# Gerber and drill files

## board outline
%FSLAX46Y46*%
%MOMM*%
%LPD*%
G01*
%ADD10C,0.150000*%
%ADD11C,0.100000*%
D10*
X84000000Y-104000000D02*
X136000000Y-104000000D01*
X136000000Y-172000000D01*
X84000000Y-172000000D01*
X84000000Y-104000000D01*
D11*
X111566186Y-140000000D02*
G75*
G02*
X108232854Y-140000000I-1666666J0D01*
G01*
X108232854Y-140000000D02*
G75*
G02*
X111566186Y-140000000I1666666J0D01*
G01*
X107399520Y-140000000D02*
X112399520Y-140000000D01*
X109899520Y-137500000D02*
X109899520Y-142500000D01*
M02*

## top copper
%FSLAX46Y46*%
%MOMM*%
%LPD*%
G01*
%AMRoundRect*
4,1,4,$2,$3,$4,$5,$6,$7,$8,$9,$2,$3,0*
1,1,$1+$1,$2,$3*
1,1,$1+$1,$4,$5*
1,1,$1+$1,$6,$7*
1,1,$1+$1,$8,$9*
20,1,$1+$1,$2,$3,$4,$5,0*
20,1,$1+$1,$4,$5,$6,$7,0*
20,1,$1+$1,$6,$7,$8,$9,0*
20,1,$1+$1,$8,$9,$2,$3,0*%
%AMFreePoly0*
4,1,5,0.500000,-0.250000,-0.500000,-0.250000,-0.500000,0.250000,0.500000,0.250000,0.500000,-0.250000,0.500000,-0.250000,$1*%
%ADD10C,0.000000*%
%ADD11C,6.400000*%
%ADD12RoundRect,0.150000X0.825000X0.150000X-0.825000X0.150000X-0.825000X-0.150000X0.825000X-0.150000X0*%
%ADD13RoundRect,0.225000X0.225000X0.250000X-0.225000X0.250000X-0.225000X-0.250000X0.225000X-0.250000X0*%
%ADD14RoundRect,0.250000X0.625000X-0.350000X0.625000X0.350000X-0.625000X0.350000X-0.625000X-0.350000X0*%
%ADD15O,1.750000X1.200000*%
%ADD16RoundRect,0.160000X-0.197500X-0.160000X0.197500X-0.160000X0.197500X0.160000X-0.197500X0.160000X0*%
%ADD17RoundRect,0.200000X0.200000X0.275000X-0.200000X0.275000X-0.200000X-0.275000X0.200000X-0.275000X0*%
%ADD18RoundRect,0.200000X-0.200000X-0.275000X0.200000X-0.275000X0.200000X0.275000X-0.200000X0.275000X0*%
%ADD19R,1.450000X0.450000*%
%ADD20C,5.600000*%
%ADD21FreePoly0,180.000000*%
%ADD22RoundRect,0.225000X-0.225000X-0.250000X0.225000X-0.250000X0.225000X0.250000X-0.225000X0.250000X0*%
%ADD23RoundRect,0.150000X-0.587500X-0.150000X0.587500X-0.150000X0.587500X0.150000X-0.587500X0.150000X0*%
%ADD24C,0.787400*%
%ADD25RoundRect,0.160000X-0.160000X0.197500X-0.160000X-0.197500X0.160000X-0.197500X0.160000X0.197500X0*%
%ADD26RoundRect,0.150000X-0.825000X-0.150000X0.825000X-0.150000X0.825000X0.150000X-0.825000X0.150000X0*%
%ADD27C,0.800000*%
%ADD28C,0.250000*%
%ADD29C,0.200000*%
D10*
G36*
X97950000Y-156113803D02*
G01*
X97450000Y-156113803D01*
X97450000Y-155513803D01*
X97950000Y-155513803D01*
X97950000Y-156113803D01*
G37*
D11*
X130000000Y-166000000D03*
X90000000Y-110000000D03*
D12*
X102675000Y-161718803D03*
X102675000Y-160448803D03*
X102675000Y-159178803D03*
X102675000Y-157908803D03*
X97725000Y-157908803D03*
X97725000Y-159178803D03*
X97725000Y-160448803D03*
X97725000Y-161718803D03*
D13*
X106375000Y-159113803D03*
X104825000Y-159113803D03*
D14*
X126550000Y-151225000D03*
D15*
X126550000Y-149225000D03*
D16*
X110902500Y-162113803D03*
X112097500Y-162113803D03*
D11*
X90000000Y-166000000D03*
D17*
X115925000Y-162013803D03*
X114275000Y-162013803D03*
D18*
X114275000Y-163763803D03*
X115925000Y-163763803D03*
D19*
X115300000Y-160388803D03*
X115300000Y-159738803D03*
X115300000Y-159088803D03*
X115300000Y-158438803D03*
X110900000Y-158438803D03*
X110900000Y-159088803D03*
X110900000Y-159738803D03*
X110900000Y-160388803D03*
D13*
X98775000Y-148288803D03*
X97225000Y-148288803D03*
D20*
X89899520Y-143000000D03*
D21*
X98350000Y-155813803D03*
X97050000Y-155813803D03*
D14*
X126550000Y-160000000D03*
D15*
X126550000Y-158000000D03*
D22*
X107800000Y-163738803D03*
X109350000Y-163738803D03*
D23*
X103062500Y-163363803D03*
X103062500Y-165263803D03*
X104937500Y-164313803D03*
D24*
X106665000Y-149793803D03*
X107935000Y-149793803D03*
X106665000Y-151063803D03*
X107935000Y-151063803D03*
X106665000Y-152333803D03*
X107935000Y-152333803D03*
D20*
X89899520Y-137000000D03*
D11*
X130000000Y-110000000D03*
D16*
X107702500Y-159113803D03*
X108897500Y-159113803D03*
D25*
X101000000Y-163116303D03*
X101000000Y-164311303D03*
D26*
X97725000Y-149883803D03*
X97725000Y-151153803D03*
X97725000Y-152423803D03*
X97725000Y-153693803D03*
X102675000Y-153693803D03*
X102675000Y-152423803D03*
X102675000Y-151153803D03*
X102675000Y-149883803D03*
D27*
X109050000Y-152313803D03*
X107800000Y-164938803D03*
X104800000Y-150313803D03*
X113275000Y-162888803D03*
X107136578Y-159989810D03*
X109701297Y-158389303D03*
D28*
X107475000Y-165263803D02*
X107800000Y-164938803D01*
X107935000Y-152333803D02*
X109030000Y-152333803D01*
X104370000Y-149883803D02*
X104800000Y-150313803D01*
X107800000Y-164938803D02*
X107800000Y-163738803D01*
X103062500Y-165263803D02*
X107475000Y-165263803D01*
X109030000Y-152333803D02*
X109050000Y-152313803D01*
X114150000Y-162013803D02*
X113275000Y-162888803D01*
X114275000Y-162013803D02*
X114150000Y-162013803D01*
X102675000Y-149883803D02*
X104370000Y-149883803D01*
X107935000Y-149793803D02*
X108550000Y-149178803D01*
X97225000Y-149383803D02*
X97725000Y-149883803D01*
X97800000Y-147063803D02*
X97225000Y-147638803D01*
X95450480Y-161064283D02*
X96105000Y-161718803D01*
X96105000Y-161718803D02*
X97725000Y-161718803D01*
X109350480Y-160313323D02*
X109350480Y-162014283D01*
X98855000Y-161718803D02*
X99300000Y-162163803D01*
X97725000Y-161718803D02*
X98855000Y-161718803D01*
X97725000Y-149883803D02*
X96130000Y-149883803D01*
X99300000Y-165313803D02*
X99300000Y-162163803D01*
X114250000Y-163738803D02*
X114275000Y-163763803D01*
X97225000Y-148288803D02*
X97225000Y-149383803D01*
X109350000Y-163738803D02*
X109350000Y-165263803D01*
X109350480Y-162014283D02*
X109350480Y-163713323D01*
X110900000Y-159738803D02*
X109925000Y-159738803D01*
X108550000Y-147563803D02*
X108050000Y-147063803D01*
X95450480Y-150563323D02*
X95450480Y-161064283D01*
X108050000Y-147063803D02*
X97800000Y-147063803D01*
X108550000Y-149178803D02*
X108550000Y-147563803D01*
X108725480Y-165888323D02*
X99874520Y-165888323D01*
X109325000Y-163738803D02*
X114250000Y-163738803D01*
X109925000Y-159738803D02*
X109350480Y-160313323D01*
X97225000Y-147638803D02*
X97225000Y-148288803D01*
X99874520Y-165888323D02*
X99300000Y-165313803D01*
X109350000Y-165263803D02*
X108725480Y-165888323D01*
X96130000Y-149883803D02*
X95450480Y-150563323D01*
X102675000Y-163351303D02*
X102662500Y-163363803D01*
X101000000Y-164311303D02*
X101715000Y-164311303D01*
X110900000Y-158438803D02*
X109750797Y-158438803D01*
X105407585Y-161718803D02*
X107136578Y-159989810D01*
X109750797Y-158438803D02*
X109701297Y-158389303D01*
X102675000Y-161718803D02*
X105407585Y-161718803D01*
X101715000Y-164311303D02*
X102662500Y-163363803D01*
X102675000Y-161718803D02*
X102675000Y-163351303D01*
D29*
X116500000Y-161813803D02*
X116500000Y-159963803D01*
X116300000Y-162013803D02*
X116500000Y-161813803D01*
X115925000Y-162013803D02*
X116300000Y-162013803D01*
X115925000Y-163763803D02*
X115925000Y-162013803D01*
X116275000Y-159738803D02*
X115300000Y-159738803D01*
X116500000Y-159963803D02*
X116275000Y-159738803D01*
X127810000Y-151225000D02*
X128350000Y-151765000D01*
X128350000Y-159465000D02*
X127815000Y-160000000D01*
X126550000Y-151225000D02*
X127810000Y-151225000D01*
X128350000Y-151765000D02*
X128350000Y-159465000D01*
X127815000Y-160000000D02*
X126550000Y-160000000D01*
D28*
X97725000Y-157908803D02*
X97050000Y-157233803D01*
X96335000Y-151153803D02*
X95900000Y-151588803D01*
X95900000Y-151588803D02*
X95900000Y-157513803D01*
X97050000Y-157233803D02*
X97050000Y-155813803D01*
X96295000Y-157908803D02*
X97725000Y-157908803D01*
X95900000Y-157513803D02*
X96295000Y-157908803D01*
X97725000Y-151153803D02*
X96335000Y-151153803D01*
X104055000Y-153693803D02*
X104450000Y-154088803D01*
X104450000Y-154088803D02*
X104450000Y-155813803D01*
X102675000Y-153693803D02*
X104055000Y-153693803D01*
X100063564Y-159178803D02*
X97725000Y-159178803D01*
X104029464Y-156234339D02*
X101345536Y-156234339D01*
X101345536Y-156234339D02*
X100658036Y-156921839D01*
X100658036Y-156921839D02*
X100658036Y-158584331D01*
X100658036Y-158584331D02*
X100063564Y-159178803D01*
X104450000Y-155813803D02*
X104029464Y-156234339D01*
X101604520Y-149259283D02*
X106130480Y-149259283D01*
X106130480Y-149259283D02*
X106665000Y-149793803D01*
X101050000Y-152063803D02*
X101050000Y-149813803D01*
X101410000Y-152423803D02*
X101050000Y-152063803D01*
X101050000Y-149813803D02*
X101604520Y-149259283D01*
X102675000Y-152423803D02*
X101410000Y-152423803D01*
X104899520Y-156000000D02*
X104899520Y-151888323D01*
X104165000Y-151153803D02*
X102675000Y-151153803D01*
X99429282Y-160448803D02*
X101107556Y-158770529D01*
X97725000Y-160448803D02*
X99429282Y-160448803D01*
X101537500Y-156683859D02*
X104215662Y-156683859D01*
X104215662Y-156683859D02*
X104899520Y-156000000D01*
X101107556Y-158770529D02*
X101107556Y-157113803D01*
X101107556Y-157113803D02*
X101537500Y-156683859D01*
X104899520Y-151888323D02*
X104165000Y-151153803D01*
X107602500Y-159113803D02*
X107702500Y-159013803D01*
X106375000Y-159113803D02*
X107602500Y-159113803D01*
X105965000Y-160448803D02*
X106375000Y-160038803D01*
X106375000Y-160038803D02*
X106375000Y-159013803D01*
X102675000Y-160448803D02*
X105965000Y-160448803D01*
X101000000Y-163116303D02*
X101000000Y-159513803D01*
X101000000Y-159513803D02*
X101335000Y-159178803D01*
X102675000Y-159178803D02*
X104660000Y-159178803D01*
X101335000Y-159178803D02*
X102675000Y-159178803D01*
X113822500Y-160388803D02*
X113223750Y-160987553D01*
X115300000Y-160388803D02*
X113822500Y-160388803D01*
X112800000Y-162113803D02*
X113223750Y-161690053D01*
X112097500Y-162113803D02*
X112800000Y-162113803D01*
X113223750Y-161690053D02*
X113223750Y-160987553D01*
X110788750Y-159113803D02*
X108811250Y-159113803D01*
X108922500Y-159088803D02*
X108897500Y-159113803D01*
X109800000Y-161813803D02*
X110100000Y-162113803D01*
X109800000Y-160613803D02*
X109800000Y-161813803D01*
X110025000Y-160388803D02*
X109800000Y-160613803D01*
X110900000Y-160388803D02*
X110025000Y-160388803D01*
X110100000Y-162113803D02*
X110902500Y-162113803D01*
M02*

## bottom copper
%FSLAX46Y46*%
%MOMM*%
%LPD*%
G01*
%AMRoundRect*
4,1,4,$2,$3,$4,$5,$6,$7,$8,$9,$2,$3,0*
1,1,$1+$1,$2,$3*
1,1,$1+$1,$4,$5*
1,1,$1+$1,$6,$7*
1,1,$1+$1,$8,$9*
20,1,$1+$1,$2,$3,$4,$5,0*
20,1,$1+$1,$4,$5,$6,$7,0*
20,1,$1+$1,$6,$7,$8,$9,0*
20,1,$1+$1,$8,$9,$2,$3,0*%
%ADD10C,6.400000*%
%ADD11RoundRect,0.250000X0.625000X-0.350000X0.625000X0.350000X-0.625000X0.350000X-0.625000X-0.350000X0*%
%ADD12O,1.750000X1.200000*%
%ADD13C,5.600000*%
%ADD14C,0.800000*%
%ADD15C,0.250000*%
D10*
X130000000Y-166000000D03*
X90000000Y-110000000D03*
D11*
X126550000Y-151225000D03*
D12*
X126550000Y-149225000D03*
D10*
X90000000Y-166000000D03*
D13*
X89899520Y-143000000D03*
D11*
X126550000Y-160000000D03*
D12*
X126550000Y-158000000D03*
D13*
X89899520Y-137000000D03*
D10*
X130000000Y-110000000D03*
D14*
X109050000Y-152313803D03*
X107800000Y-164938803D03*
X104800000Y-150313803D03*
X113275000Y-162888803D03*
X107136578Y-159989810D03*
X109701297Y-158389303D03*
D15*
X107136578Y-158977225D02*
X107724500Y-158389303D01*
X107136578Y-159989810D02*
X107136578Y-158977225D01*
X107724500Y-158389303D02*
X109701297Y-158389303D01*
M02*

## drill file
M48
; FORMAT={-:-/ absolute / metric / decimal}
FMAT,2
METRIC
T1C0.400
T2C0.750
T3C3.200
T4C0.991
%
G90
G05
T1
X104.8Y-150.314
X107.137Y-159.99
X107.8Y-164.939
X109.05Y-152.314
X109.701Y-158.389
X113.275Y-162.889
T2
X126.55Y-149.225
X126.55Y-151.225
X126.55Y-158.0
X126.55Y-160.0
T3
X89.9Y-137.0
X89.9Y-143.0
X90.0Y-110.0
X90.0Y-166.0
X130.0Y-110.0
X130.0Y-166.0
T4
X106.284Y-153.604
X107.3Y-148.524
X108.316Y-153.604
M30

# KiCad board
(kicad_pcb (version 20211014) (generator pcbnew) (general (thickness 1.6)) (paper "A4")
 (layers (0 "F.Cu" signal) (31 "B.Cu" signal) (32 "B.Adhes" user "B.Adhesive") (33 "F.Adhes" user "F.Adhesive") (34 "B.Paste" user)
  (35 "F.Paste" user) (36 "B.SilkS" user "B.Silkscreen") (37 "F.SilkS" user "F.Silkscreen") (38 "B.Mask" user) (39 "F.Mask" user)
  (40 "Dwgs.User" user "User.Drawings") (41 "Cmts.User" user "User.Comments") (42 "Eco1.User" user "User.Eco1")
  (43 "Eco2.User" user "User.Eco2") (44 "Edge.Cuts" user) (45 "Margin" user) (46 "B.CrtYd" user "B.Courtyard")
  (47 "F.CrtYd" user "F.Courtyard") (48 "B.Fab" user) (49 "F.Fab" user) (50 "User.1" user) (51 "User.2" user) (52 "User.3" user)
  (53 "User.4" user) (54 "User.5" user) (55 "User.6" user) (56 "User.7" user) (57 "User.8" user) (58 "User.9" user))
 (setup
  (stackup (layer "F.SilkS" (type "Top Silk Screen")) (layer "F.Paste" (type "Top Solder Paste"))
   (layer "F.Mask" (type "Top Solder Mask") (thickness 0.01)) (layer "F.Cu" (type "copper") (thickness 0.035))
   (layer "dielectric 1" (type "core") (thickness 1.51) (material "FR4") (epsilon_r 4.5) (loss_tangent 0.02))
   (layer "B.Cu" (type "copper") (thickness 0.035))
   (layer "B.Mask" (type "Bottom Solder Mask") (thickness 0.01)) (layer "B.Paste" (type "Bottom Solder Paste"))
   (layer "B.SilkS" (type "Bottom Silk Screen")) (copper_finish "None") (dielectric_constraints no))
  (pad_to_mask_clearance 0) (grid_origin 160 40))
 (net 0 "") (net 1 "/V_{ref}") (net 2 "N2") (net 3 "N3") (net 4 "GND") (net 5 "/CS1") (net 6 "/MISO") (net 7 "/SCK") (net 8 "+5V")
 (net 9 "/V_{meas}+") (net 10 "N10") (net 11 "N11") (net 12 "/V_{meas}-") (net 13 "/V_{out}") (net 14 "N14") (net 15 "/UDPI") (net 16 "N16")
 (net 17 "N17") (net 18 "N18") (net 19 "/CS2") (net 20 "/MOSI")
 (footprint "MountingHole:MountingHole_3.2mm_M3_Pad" (layer "F.Cu") (at 130 166)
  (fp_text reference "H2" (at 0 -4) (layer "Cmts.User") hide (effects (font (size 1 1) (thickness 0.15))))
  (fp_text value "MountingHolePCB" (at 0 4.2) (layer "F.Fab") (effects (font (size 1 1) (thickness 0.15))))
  (pad "1" thru_hole circle locked (at 0 0) (size 6.4 6.4) (drill 3.2) (layers *.Cu *.Mask)))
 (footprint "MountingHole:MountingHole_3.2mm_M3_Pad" (layer "F.Cu") (at 90 110)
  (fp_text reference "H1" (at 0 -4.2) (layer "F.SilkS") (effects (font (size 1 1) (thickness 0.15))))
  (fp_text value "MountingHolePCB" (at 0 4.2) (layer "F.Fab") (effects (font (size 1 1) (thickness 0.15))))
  (pad "1" thru_hole circle locked (at 0 0) (size 6.4 6.4) (drill 3.2) (layers *.Cu *.Mask)))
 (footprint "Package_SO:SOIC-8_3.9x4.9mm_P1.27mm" (layer "F.Cu") (at 100.2 159.813803 180)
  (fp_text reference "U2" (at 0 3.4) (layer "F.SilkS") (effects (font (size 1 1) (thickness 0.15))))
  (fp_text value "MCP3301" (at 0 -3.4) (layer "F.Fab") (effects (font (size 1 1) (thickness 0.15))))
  (pad "1" smd roundrect locked (at -2.475 -1.905 180) (size 1.95 0.6) (layers "F.Cu" "F.Paste" "F.Mask") (roundrect_rratio 0.25)
   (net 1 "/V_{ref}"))
  (pad "2" smd roundrect locked (at -2.475 -0.635 180) (size 1.95 0.6) (layers "F.Cu" "F.Paste" "F.Mask") (roundrect_rratio 0.25)
   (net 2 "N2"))
  (pad "3" smd roundrect locked (at -2.475 0.635 180) (size 1.95 0.6) (layers "F.Cu" "F.Paste" "F.Mask") (roundrect_rratio 0.25)
   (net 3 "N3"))
  (pad "4" smd roundrect locked (at -2.475 1.905 180) (size 1.95 0.6) (layers "F.Cu" "F.Paste" "F.Mask") (roundrect_rratio 0.25)
   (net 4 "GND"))
  (pad "5" smd roundrect locked (at 2.475 1.905 180) (size 1.95 0.6) (layers "F.Cu" "F.Paste" "F.Mask") (roundrect_rratio 0.25)
   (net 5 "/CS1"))
  (pad "6" smd roundrect locked (at 2.475 0.635 180) (size 1.95 0.6) (layers "F.Cu" "F.Paste" "F.Mask") (roundrect_rratio 0.25)
   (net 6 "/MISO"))
  (pad "7" smd roundrect locked (at 2.475 -0.635 180) (size 1.95 0.6) (layers "F.Cu" "F.Paste" "F.Mask") (roundrect_rratio 0.25)
   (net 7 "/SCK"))
  (pad "8" smd roundrect locked (at 2.475 -1.905 180) (size 1.95 0.6) (layers "F.Cu" "F.Paste" "F.Mask") (roundrect_rratio 0.25)
   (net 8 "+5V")))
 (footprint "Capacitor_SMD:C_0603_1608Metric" (layer "F.Cu") (at 105.6 159.113803 180)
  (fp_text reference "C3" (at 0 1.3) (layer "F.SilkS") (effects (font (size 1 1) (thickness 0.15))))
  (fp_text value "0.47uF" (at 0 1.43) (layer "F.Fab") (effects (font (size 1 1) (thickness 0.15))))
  (pad "1" smd roundrect locked (at -0.775 0 180) (size 0.9 0.95) (layers "F.Cu" "F.Paste" "F.Mask") (roundrect_rratio 0.25) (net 2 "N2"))
  (pad "2" smd roundrect locked (at 0.775 0 180) (size 0.9 0.95) (layers "F.Cu" "F.Paste" "F.Mask") (roundrect_rratio 0.25) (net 3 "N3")))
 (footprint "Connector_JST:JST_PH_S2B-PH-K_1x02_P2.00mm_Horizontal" (layer "F.Cu") (at 126.55 151.225 90)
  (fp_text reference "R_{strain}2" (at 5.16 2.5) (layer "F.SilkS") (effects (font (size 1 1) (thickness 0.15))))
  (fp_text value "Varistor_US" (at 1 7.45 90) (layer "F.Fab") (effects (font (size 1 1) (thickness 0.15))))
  (pad "1" thru_hole roundrect locked (at 0 0 90) (size 1.2 1.75) (drill 0.75) (layers *.Cu *.Mask) (roundrect_rratio 0.208333)
   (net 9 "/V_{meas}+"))
  (pad "2" thru_hole oval locked (at 2 0 90) (size 1.2 1.75) (drill 0.75) (layers *.Cu *.Mask) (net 4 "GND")))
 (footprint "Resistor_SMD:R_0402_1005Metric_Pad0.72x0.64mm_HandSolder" (layer "F.Cu") (at 111.5 162.113803)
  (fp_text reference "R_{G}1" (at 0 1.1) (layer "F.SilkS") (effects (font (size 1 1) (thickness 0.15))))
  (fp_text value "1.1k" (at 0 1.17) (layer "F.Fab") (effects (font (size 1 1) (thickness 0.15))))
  (pad "1" smd roundrect locked (at -0.5975 0) (size 0.715 0.64) (layers "F.Cu" "F.Paste" "F.Mask") (roundrect_rratio 0.25) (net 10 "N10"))
  (pad "2" smd roundrect locked (at 0.5975 0) (size 0.715 0.64) (layers "F.Cu" "F.Paste" "F.Mask") (roundrect_rratio 0.25) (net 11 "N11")))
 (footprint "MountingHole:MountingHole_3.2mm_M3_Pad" (layer "F.Cu") (at 90 166)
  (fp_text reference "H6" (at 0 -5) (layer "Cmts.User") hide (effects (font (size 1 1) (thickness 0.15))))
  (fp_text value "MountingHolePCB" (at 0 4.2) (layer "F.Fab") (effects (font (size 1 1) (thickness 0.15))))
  (pad "1" thru_hole circle locked (at 0 0) (size 6.4 6.4) (drill 3.2) (layers *.Cu *.Mask)))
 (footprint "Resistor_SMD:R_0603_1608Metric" (layer "F.Cu") (at 115.1 162.013803 180)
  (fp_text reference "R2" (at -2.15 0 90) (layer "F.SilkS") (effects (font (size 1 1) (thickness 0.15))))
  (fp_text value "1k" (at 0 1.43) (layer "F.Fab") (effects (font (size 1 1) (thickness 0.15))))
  (pad "1" smd roundrect locked (at -0.825 0 180) (size 0.8 0.95) (layers "F.Cu" "F.Paste" "F.Mask") (roundrect_rratio 0.25)
   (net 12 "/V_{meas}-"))
  (pad "2" smd roundrect locked (at 0.825 0 180) (size 0.8 0.95) (layers "F.Cu" "F.Paste" "F.Mask") (roundrect_rratio 0.25) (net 4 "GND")))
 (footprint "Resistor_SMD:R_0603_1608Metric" (layer "F.Cu") (at 115.1 163.763803)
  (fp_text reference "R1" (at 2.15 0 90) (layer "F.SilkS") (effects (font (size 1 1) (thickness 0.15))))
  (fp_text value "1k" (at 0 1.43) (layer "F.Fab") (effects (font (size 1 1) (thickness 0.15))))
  (pad "1" smd roundrect locked (at -0.825 0) (size 0.8 0.95) (layers "F.Cu" "F.Paste" "F.Mask") (roundrect_rratio 0.25) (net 8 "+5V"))
  (pad "2" smd roundrect locked (at 0.825 0) (size 0.8 0.95) (layers "F.Cu" "F.Paste" "F.Mask") (roundrect_rratio 0.25)
   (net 12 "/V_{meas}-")))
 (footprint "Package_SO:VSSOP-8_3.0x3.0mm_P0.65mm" (layer "F.Cu") (at 113.1 159.413803 180)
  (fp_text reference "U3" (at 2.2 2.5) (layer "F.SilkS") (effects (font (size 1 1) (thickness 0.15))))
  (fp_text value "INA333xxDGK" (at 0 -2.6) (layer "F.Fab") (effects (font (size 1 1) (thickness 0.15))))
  (pad "1" smd rect locked (at -2.2 -0.975 90) (size 0.45 1.45) (layers "F.Cu" "F.Paste" "F.Mask") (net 11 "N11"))
  (pad "2" smd rect locked (at -2.2 -0.325 90) (size 0.45 1.45) (layers "F.Cu" "F.Paste" "F.Mask") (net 12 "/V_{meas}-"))
  (pad "3" smd rect locked (at -2.2 0.325 90) (size 0.45 1.45) (layers "F.Cu" "F.Paste" "F.Mask") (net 9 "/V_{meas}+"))
  (pad "4" smd rect locked (at -2.2 0.975 90) (size 0.45 1.45) (layers "F.Cu" "F.Paste" "F.Mask") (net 4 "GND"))
  (pad "5" smd rect locked (at 2.2 0.975 90) (size 0.45 1.45) (layers "F.Cu" "F.Paste" "F.Mask") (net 1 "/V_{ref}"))
  (pad "6" smd rect locked (at 2.2 0.325 90) (size 0.45 1.45) (layers "F.Cu" "F.Paste" "F.Mask") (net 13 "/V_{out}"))
  (pad "7" smd rect locked (at 2.2 -0.325 90) (size 0.45 1.45) (layers "F.Cu" "F.Paste" "F.Mask") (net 8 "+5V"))
  (pad "8" smd rect locked (at 2.2 -0.975 90) (size 0.45 1.45) (layers "F.Cu" "F.Paste" "F.Mask") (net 10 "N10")))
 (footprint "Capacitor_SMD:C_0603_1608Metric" (layer "F.Cu") (at 98 148.288803 180)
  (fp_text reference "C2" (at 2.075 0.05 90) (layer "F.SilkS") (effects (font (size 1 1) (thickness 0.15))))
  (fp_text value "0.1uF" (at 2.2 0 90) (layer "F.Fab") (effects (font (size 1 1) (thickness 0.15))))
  (pad "1" smd roundrect locked (at -0.775 0 180) (size 0.9 0.95) (layers "F.Cu" "F.Paste" "F.Mask") (roundrect_rratio 0.25) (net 4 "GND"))
  (pad "2" smd roundrect locked (at 0.775 0 180) (size 0.9 0.95) (layers "F.Cu" "F.Paste" "F.Mask") (roundrect_rratio 0.25) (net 8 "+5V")))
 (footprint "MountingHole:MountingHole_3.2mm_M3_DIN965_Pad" (layer "F.Cu") (at 89.89952 143)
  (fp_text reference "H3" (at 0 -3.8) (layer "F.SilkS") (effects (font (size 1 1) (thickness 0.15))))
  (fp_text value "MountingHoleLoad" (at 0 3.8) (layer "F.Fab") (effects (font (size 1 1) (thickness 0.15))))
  (pad "1" thru_hole circle locked (at 0 0) (size 5.6 5.6) (drill 3.2) (layers *.Cu *.Mask)))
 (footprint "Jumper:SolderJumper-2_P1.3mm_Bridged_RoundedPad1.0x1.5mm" (layer "F.Cu") (at 97.7 155.813803 180)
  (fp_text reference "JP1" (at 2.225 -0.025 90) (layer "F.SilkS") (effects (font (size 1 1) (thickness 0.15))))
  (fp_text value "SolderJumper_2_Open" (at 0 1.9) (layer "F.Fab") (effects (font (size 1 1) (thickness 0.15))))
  (fp_poly (pts (xy 0.25 -0.3) (xy -0.25 -0.3) (xy -0.25 0.3) (xy 0.25 0.3)) (layer "F.Cu") (width 0) (fill solid))
  (pad "1" smd custom locked (at -0.65 0 180) (size 1 0.5) (layers "F.Cu" "F.Mask") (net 4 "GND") (zone_connect 2)
   (options (clearance outline) (anchor rect)) (primitives))
  (pad "2" smd custom locked (at 0.65 0 180) (size 1 0.5) (layers "F.Cu" "F.Mask") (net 5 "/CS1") (zone_connect 2)
   (options (clearance outline) (anchor rect)) (primitives)))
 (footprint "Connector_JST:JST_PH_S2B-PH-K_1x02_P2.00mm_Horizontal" (layer "F.Cu") (at 126.55 160 90)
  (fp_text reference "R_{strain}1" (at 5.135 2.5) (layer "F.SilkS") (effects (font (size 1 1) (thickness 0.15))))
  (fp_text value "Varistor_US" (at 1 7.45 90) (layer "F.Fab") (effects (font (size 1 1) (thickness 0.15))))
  (pad "1" thru_hole roundrect locked (at 0 0 90) (size 1.2 1.75) (drill 0.75) (layers *.Cu *.Mask) (roundrect_rratio 0.208333)
   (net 9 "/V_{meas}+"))
  (pad "2" thru_hole oval locked (at 2 0 90) (size 1.2 1.75) (drill 0.75) (layers *.Cu *.Mask) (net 8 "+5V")))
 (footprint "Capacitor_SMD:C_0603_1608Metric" (layer "F.Cu") (at 108.575 163.738803)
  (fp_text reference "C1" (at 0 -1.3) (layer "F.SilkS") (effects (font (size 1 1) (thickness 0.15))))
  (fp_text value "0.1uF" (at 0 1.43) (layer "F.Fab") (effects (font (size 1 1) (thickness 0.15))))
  (pad "1" smd roundrect locked (at -0.775 0) (size 0.9 0.95) (layers "F.Cu" "F.Paste" "F.Mask") (roundrect_rratio 0.25) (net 4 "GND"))
  (pad "2" smd roundrect locked (at 0.775 0) (size 0.9 0.95) (layers "F.Cu" "F.Paste" "F.Mask") (roundrect_rratio 0.25) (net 8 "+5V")))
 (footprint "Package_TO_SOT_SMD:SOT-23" (layer "F.Cu") (at 104 164.313803)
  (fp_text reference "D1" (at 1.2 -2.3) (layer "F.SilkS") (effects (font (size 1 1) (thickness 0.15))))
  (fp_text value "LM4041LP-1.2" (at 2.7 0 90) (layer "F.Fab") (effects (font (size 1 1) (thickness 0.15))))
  (pad "1" smd roundrect locked (at -0.9375 -0.95) (size 1.475 0.6) (layers "F.Cu" "F.Paste" "F.Mask") (roundrect_rratio 0.25)
   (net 1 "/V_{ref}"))
  (pad "2" smd roundrect locked (at -0.9375 0.95) (size 1.475 0.6) (layers "F.Cu" "F.Paste" "F.Mask") (roundrect_rratio 0.25) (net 4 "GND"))
  (pad "3" smd roundrect locked (at 0.9375 0) (size 1.475 0.6) (layers "F.Cu" "F.Paste" "F.Mask") (roundrect_rratio 0.25) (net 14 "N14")))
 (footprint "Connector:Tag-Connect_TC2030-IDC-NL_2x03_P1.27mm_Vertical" (layer "F.Cu") (at 107.3 151.063803 -90)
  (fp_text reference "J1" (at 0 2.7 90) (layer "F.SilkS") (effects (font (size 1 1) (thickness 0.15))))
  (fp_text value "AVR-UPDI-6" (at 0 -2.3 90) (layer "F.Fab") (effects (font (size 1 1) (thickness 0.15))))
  (pad "" np_thru_hole circle locked (at -2.54 0 270) (size 0.9906 0.9906) (drill 0.9906) (layers *.Cu *.Mask))
  (pad "" np_thru_hole circle locked (at 2.54 1.016 270) (size 0.9906 0.9906) (drill 0.9906) (layers *.Cu *.Mask))
  (pad "" np_thru_hole circle locked (at 2.54 -1.016 270) (size 0.9906 0.9906) (drill 0.9906) (layers *.Cu *.Mask))
  (pad "1" connect circle locked (at -1.27 0.635 270) (size 0.7874 0.7874) (layers "F.Cu" "F.Mask") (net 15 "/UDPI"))
  (pad "2" connect circle locked (at -1.27 -0.635 270) (size 0.7874 0.7874) (layers "F.Cu" "F.Mask") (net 8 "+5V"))
  (pad "3" connect circle locked (at 0 0.635 270) (size 0.7874 0.7874) (layers "F.Cu" "F.Mask") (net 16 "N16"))
  (pad "4" connect circle locked (at 0 -0.635 270) (size 0.7874 0.7874) (layers "F.Cu" "F.Mask") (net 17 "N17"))
  (pad "5" connect circle locked (at 1.27 0.635 270) (size 0.7874 0.7874) (layers "F.Cu" "F.Mask") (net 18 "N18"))
  (pad "6" connect circle locked (at 1.27 -0.635 270) (size 0.7874 0.7874) (layers "F.Cu" "F.Mask") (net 4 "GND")))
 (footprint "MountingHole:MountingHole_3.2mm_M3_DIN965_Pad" (layer "F.Cu") (at 89.89952 137)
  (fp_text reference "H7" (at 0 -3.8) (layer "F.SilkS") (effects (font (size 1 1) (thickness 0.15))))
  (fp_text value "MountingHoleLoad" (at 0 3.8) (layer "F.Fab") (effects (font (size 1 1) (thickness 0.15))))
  (pad "1" thru_hole circle locked (at 0 0) (size 5.6 5.6) (drill 3.2) (layers *.Cu *.Mask)))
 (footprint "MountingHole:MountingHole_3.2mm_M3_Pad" (layer "F.Cu") (at 130 110)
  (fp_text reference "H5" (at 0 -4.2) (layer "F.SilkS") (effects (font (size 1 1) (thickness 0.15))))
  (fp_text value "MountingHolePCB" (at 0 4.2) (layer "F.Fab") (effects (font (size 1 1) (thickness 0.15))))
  (pad "1" thru_hole circle locked (at 0 0) (size 6.4 6.4) (drill 3.2) (layers *.Cu *.Mask)))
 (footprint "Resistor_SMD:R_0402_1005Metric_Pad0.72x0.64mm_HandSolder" (layer "F.Cu") (at 108.3 159.113803)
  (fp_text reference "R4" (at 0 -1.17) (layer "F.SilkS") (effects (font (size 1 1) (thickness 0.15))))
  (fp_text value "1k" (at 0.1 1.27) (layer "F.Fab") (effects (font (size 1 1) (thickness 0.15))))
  (pad "1" smd roundrect locked (at -0.5975 0) (size 0.715 0.64) (layers "F.Cu" "F.Paste" "F.Mask") (roundrect_rratio 0.25) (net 2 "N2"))
  (pad "2" smd roundrect locked (at 0.5975 0) (size 0.715 0.64) (layers "F.Cu" "F.Paste" "F.Mask") (roundrect_rratio 0.25)
   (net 13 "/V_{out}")))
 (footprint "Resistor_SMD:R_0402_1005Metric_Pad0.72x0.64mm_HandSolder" (layer "F.Cu") (at 101 163.713803 -90)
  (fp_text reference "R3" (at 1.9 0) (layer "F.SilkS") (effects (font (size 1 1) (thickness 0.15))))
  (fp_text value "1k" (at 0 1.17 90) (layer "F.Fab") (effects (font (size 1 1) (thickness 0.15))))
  (pad "1" smd roundrect locked (at -0.5975 0 270) (size 0.715 0.64) (layers "F.Cu" "F.Paste" "F.Mask") (roundrect_rratio 0.25) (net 3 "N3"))
  (pad "2" smd roundrect locked (at 0.5975 0 270) (size 0.715 0.64) (layers "F.Cu" "F.Paste" "F.Mask") (roundrect_rratio 0.25)
   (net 1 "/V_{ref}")))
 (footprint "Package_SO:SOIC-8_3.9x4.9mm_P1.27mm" (layer "F.Cu") (at 100.2 151.788803)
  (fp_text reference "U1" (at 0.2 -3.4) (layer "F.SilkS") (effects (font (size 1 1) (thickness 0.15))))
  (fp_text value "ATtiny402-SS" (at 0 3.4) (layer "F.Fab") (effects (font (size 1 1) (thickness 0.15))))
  (pad "1" smd roundrect locked (at -2.475 -1.905) (size 1.95 0.6) (layers "F.Cu" "F.Paste" "F.Mask") (roundrect_rratio 0.25) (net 8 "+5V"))
  (pad "2" smd roundrect locked (at -2.475 -0.635) (size 1.95 0.6) (layers "F.Cu" "F.Paste" "F.Mask") (roundrect_rratio 0.25) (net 5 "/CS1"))
  (pad "3" smd roundrect locked (at -2.475 0.635) (size 1.95 0.6) (layers "F.Cu" "F.Paste" "F.Mask") (roundrect_rratio 0.25) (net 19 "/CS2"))
  (pad "4" smd roundrect locked (at -2.475 1.905) (size 1.95 0.6) (layers "F.Cu" "F.Paste" "F.Mask") (roundrect_rratio 0.25)
   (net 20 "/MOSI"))
  (pad "5" smd roundrect locked (at 2.475 1.905) (size 1.95 0.6) (layers "F.Cu" "F.Paste" "F.Mask") (roundrect_rratio 0.25) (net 6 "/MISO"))
  (pad "6" smd roundrect locked (at 2.475 0.635) (size 1.95 0.6) (layers "F.Cu" "F.Paste" "F.Mask") (roundrect_rratio 0.25) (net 15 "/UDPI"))
  (pad "7" smd roundrect locked (at 2.475 -0.635) (size 1.95 0.6) (layers "F.Cu" "F.Paste" "F.Mask") (roundrect_rratio 0.25) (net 7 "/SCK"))
  (pad "8" smd roundrect locked (at 2.475 -1.905) (size 1.95 0.6) (layers "F.Cu" "F.Paste" "F.Mask") (roundrect_rratio 0.25) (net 4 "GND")))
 (gr_rect (start 84 104) (end 136 172) (layer "Edge.Cuts") (width 0.15) (fill none))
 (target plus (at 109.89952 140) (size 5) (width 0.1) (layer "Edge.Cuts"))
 (segment (start 107.475 165.263803) (end 107.8 164.938803) (width 0.25) (layer "F.Cu") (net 4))
 (segment (start 107.935 152.333803) (end 109.03 152.333803) (width 0.25) (layer "F.Cu") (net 4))
 (segment (start 104.37 149.883803) (end 104.8 150.313803) (width 0.25) (layer "F.Cu") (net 4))
 (segment (start 107.8 164.938803) (end 107.8 163.738803) (width 0.25) (layer "F.Cu") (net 4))
 (segment (start 103.0625 165.263803) (end 107.475 165.263803) (width 0.25) (layer "F.Cu") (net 4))
 (segment (start 109.03 152.333803) (end 109.05 152.313803) (width 0.25) (layer "F.Cu") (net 4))
 (segment (start 114.15 162.013803) (end 113.275 162.888803) (width 0.25) (layer "F.Cu") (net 4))
 (segment (start 114.275 162.013803) (end 114.15 162.013803) (width 0.25) (layer "F.Cu") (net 4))
 (segment (start 102.675 149.883803) (end 104.37 149.883803) (width 0.25) (layer "F.Cu") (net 4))
 (via (at 109.05 152.313803) (size 0.8) (drill 0.4) (layers "F.Cu" "B.Cu") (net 4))
 (via (at 107.8 164.938803) (size 0.8) (drill 0.4) (layers "F.Cu" "B.Cu") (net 4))
 (via (at 104.8 150.313803) (size 0.8) (drill 0.4) (layers "F.Cu" "B.Cu") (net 4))
 (via (at 113.275 162.888803) (size 0.8) (drill 0.4) (layers "F.Cu" "B.Cu") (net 4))
 (segment (start 107.935 149.793803) (end 108.55 149.178803) (width 0.25) (layer "F.Cu") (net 8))
 (segment (start 97.225 149.383803) (end 97.725 149.883803) (width 0.25) (layer "F.Cu") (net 8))
 (segment (start 97.8 147.063803) (end 97.225 147.638803) (width 0.25) (layer "F.Cu") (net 8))
 (segment (start 95.45048 161.064283) (end 96.105 161.718803) (width 0.25) (layer "F.Cu") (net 8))
 (segment (start 96.105 161.718803) (end 97.725 161.718803) (width 0.25) (layer "F.Cu") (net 8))
 (segment (start 109.35048 160.313323) (end 109.35048 162.014283) (width 0.25) (layer "F.Cu") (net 8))
 (segment (start 98.855 161.718803) (end 99.3 162.163803) (width 0.25) (layer "F.Cu") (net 8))
 (segment (start 97.725 161.718803) (end 98.855 161.718803) (width 0.25) (layer "F.Cu") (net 8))
 (segment (start 97.725 149.883803) (end 96.13 149.883803) (width 0.25) (layer "F.Cu") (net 8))
 (segment (start 99.3 165.313803) (end 99.3 162.163803) (width 0.25) (layer "F.Cu") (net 8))
 (segment (start 114.25 163.738803) (end 114.275 163.763803) (width 0.25) (layer "F.Cu") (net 8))
 (segment (start 97.225 148.288803) (end 97.225 149.383803) (width 0.25) (layer "F.Cu") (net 8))
 (segment (start 109.35 163.738803) (end 109.35 165.263803) (width 0.25) (layer "F.Cu") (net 8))
 (segment (start 109.35048 162.014283) (end 109.35048 163.713323) (width 0.25) (layer "F.Cu") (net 8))
 (segment (start 110.9 159.738803) (end 109.925 159.738803) (width 0.25) (layer "F.Cu") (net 8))
 (segment (start 108.55 147.563803) (end 108.05 147.063803) (width 0.25) (layer "F.Cu") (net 8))
 (segment (start 95.45048 150.563323) (end 95.45048 161.064283) (width 0.25) (layer "F.Cu") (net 8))
 (segment (start 108.05 147.063803) (end 97.8 147.063803) (width 0.25) (layer "F.Cu") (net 8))
 (segment (start 108.55 149.178803) (end 108.55 147.563803) (width 0.25) (layer "F.Cu") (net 8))
 (segment (start 108.72548 165.888323) (end 99.87452 165.888323) (width 0.25) (layer "F.Cu") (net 8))
 (segment (start 109.325 163.738803) (end 114.25 163.738803) (width 0.25) (layer "F.Cu") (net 8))
 (segment (start 109.925 159.738803) (end 109.35048 160.313323) (width 0.25) (layer "F.Cu") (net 8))
 (segment (start 97.225 147.638803) (end 97.225 148.288803) (width 0.25) (layer "F.Cu") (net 8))
 (segment (start 99.87452 165.888323) (end 99.3 165.313803) (width 0.25) (layer "F.Cu") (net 8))
 (segment (start 109.35 165.263803) (end 108.72548 165.888323) (width 0.25) (layer "F.Cu") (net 8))
 (segment (start 96.13 149.883803) (end 95.45048 150.563323) (width 0.25) (layer "F.Cu") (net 8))
 (segment (start 102.675 163.351303) (end 102.6625 163.363803) (width 0.25) (layer "F.Cu") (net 1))
 (segment (start 101 164.311303) (end 101.715 164.311303) (width 0.25) (layer "F.Cu") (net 1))
 (segment (start 110.9 158.438803) (end 109.750797 158.438803) (width 0.25) (layer "F.Cu") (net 1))
 (segment (start 105.407585 161.718803) (end 107.136578 159.98981) (width 0.25) (layer "F.Cu") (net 1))
 (segment (start 109.750797 158.438803) (end 109.701297 158.389303) (width 0.25) (layer "F.Cu") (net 1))
 (segment (start 102.675 161.718803) (end 105.407585 161.718803) (width 0.25) (layer "F.Cu") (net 1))
 (segment (start 101.715 164.311303) (end 102.6625 163.363803) (width 0.25) (layer "F.Cu") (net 1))
 (segment (start 102.675 161.718803) (end 102.675 163.351303) (width 0.25) (layer "F.Cu") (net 1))
 (via (at 107.136578 159.98981) (size 0.8) (drill 0.4) (layers "F.Cu" "B.Cu") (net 1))
 (via (at 109.701297 158.389303) (size 0.8) (drill 0.4) (layers "F.Cu" "B.Cu") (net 1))
 (segment (start 107.136578 158.977225) (end 107.7245 158.389303) (width 0.25) (layer "B.Cu") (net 1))
 (segment (start 107.136578 159.98981) (end 107.136578 158.977225) (width 0.25) (layer "B.Cu") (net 1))
 (segment (start 107.7245 158.389303) (end 109.701297 158.389303) (width 0.25) (layer "B.Cu") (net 1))
 (segment (start 116.5 161.813803) (end 116.5 159.963803) (width 0.2) (layer "F.Cu") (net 12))
 (segment (start 116.3 162.013803) (end 116.5 161.813803) (width 0.2) (layer "F.Cu") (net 12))
 (segment (start 115.925 162.013803) (end 116.3 162.013803) (width 0.2) (layer "F.Cu") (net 12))
 (segment (start 115.925 163.763803) (end 115.925 162.013803) (width 0.2) (layer "F.Cu") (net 12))
 (segment (start 116.275 159.738803) (end 115.3 159.738803) (width 0.2) (layer "F.Cu") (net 12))
 (segment (start 116.5 159.963803) (end 116.275 159.738803) (width 0.2) (layer "F.Cu") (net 12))
 (segment (start 127.81 151.225) (end 128.35 151.765) (width 0.2) (layer "F.Cu") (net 9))
 (segment (start 128.35 159.465) (end 127.815 160) (width 0.2) (layer "F.Cu") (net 9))
 (segment (start 126.55 151.225) (end 127.81 151.225) (width 0.2) (layer "F.Cu") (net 9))
 (segment (start 128.35 151.765) (end 128.35 159.465) (width 0.2) (layer "F.Cu") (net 9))
 (segment (start 127.815 160) (end 126.55 160) (width 0.2) (layer "F.Cu") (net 9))
 (segment (start 97.725 157.908803) (end 97.05 157.233803) (width 0.25) (layer "F.Cu") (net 5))
 (segment (start 96.335 151.153803) (end 95.9 151.588803) (width 0.25) (layer "F.Cu") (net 5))
 (segment (start 95.9 151.588803) (end 95.9 157.513803) (width 0.25) (layer "F.Cu") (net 5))
 (segment (start 97.05 157.233803) (end 97.05 155.813803) (width 0.25) (layer "F.Cu") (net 5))
 (segment (start 96.295 157.908803) (end 97.725 157.908803) (width 0.25) (layer "F.Cu") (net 5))
 (segment (start 95.9 157.513803) (end 96.295 157.908803) (width 0.25) (layer "F.Cu") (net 5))
 (segment (start 97.725 151.153803) (end 96.335 151.153803) (width 0.25) (layer "F.Cu") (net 5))
 (segment (start 104.055 153.693803) (end 104.45 154.088803) (width 0.25) (layer "F.Cu") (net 6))
 (segment (start 104.45 154.088803) (end 104.45 155.813803) (width 0.25) (layer "F.Cu") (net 6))
 (segment (start 102.675 153.693803) (end 104.055 153.693803) (width 0.25) (layer "F.Cu") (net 6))
 (segment (start 100.063564 159.178803) (end 97.725 159.178803) (width 0.25) (layer "F.Cu") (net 6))
 (segment (start 104.029464 156.234339) (end 101.345536 156.234339) (width 0.25) (layer "F.Cu") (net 6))
 (segment (start 101.345536 156.234339) (end 100.658036 156.921839) (width 0.25) (layer "F.Cu") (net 6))
 (segment (start 100.658036 156.921839) (end 100.658036 158.584331) (width 0.25) (layer "F.Cu") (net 6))
 (segment (start 100.658036 158.584331) (end 100.063564 159.178803) (width 0.25) (layer "F.Cu") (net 6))
 (segment (start 104.45 155.813803) (end 104.029464 156.234339) (width 0.25) (layer "F.Cu") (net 6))
 (segment (start 101.60452 149.259283) (end 106.13048 149.259283) (width 0.25) (layer "F.Cu") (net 15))
 (segment (start 106.13048 149.259283) (end 106.665 149.793803) (width 0.25) (layer "F.Cu") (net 15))
 (segment (start 101.05 152.063803) (end 101.05 149.813803) (width 0.25) (layer "F.Cu") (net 15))
 (segment (start 101.41 152.423803) (end 101.05 152.063803) (width 0.25) (layer "F.Cu") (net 15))
 (segment (start 101.05 149.813803) (end 101.60452 149.259283) (width 0.25) (layer "F.Cu") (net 15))
 (segment (start 102.675 152.423803) (end 101.41 152.423803) (width 0.25) (layer "F.Cu") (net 15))
 (segment (start 104.89952 156) (end 104.89952 151.888323) (width 0.25) (layer "F.Cu") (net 7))
 (segment (start 104.165 151.153803) (end 102.675 151.153803) (width 0.25) (layer "F.Cu") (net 7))
 (segment (start 99.429282 160.448803) (end 101.107556 158.770529) (width 0.25) (layer "F.Cu") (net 7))
 (segment (start 97.725 160.448803) (end 99.429282 160.448803) (width 0.25) (layer "F.Cu") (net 7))
 (segment (start 101.5375 156.683859) (end 104.215662 156.683859) (width 0.25) (layer "F.Cu") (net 7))
 (segment (start 104.215662 156.683859) (end 104.89952 156) (width 0.25) (layer "F.Cu") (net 7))
 (segment (start 101.107556 158.770529) (end 101.107556 157.113803) (width 0.25) (layer "F.Cu") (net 7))
 (segment (start 101.107556 157.113803) (end 101.5375 156.683859) (width 0.25) (layer "F.Cu") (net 7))
 (segment (start 104.89952 151.888323) (end 104.165 151.153803) (width 0.25) (layer "F.Cu") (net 7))
 (segment (start 107.6025 159.113803) (end 107.7025 159.013803) (width 0.25) (layer "F.Cu") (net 2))
 (segment (start 106.375 159.113803) (end 107.6025 159.113803) (width 0.25) (layer "F.Cu") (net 2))
 (segment (start 105.965 160.448803) (end 106.375 160.038803) (width 0.25) (layer "F.Cu") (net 2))
 (segment (start 106.375 160.038803) (end 106.375 159.013803) (width 0.25) (layer "F.Cu") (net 2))
 (segment (start 102.675 160.448803) (end 105.965 160.448803) (width 0.25) (layer "F.Cu") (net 2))
 (segment (start 101 163.116303) (end 101 159.513803) (width 0.25) (layer "F.Cu") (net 3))
 (segment (start 101 159.513803) (end 101.335 159.178803) (width 0.25) (layer "F.Cu") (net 3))
 (segment (start 102.675 159.178803) (end 104.66 159.178803) (width 0.25) (layer "F.Cu") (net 3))
 (segment (start 101.335 159.178803) (end 102.675 159.178803) (width 0.25) (layer "F.Cu") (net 3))
 (segment (start 113.8225 160.388803) (end 113.22375 160.987553) (width 0.25) (layer "F.Cu") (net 11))
 (segment (start 115.3 160.388803) (end 113.8225 160.388803) (width 0.25) (layer "F.Cu") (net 11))
 (segment (start 112.8 162.113803) (end 113.22375 161.690053) (width 0.25) (layer "F.Cu") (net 11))
 (segment (start 112.0975 162.113803) (end 112.8 162.113803) (width 0.25) (layer "F.Cu") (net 11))
 (segment (start 113.22375 161.690053) (end 113.22375 160.987553) (width 0.25) (layer "F.Cu") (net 11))
 (segment (start 110.78875 159.113803) (end 108.81125 159.113803) (width 0.25) (layer "F.Cu") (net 13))
 (segment (start 108.9225 159.088803) (end 108.8975 159.113803) (width 0.25) (layer "F.Cu") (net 13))
 (segment (start 109.8 161.813803) (end 110.1 162.113803) (width 0.25) (layer "F.Cu") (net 10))
 (segment (start 109.8 160.613803) (end 109.8 161.813803) (width 0.25) (layer "F.Cu") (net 10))
 (segment (start 110.025 160.388803) (end 109.8 160.613803) (width 0.25) (layer "F.Cu") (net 10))
 (segment (start 110.9 160.388803) (end 110.025 160.388803) (width 0.25) (layer "F.Cu") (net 10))
 (segment (start 110.1 162.113803) (end 110.9025 162.113803) (width 0.25) (layer "F.Cu") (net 10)))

